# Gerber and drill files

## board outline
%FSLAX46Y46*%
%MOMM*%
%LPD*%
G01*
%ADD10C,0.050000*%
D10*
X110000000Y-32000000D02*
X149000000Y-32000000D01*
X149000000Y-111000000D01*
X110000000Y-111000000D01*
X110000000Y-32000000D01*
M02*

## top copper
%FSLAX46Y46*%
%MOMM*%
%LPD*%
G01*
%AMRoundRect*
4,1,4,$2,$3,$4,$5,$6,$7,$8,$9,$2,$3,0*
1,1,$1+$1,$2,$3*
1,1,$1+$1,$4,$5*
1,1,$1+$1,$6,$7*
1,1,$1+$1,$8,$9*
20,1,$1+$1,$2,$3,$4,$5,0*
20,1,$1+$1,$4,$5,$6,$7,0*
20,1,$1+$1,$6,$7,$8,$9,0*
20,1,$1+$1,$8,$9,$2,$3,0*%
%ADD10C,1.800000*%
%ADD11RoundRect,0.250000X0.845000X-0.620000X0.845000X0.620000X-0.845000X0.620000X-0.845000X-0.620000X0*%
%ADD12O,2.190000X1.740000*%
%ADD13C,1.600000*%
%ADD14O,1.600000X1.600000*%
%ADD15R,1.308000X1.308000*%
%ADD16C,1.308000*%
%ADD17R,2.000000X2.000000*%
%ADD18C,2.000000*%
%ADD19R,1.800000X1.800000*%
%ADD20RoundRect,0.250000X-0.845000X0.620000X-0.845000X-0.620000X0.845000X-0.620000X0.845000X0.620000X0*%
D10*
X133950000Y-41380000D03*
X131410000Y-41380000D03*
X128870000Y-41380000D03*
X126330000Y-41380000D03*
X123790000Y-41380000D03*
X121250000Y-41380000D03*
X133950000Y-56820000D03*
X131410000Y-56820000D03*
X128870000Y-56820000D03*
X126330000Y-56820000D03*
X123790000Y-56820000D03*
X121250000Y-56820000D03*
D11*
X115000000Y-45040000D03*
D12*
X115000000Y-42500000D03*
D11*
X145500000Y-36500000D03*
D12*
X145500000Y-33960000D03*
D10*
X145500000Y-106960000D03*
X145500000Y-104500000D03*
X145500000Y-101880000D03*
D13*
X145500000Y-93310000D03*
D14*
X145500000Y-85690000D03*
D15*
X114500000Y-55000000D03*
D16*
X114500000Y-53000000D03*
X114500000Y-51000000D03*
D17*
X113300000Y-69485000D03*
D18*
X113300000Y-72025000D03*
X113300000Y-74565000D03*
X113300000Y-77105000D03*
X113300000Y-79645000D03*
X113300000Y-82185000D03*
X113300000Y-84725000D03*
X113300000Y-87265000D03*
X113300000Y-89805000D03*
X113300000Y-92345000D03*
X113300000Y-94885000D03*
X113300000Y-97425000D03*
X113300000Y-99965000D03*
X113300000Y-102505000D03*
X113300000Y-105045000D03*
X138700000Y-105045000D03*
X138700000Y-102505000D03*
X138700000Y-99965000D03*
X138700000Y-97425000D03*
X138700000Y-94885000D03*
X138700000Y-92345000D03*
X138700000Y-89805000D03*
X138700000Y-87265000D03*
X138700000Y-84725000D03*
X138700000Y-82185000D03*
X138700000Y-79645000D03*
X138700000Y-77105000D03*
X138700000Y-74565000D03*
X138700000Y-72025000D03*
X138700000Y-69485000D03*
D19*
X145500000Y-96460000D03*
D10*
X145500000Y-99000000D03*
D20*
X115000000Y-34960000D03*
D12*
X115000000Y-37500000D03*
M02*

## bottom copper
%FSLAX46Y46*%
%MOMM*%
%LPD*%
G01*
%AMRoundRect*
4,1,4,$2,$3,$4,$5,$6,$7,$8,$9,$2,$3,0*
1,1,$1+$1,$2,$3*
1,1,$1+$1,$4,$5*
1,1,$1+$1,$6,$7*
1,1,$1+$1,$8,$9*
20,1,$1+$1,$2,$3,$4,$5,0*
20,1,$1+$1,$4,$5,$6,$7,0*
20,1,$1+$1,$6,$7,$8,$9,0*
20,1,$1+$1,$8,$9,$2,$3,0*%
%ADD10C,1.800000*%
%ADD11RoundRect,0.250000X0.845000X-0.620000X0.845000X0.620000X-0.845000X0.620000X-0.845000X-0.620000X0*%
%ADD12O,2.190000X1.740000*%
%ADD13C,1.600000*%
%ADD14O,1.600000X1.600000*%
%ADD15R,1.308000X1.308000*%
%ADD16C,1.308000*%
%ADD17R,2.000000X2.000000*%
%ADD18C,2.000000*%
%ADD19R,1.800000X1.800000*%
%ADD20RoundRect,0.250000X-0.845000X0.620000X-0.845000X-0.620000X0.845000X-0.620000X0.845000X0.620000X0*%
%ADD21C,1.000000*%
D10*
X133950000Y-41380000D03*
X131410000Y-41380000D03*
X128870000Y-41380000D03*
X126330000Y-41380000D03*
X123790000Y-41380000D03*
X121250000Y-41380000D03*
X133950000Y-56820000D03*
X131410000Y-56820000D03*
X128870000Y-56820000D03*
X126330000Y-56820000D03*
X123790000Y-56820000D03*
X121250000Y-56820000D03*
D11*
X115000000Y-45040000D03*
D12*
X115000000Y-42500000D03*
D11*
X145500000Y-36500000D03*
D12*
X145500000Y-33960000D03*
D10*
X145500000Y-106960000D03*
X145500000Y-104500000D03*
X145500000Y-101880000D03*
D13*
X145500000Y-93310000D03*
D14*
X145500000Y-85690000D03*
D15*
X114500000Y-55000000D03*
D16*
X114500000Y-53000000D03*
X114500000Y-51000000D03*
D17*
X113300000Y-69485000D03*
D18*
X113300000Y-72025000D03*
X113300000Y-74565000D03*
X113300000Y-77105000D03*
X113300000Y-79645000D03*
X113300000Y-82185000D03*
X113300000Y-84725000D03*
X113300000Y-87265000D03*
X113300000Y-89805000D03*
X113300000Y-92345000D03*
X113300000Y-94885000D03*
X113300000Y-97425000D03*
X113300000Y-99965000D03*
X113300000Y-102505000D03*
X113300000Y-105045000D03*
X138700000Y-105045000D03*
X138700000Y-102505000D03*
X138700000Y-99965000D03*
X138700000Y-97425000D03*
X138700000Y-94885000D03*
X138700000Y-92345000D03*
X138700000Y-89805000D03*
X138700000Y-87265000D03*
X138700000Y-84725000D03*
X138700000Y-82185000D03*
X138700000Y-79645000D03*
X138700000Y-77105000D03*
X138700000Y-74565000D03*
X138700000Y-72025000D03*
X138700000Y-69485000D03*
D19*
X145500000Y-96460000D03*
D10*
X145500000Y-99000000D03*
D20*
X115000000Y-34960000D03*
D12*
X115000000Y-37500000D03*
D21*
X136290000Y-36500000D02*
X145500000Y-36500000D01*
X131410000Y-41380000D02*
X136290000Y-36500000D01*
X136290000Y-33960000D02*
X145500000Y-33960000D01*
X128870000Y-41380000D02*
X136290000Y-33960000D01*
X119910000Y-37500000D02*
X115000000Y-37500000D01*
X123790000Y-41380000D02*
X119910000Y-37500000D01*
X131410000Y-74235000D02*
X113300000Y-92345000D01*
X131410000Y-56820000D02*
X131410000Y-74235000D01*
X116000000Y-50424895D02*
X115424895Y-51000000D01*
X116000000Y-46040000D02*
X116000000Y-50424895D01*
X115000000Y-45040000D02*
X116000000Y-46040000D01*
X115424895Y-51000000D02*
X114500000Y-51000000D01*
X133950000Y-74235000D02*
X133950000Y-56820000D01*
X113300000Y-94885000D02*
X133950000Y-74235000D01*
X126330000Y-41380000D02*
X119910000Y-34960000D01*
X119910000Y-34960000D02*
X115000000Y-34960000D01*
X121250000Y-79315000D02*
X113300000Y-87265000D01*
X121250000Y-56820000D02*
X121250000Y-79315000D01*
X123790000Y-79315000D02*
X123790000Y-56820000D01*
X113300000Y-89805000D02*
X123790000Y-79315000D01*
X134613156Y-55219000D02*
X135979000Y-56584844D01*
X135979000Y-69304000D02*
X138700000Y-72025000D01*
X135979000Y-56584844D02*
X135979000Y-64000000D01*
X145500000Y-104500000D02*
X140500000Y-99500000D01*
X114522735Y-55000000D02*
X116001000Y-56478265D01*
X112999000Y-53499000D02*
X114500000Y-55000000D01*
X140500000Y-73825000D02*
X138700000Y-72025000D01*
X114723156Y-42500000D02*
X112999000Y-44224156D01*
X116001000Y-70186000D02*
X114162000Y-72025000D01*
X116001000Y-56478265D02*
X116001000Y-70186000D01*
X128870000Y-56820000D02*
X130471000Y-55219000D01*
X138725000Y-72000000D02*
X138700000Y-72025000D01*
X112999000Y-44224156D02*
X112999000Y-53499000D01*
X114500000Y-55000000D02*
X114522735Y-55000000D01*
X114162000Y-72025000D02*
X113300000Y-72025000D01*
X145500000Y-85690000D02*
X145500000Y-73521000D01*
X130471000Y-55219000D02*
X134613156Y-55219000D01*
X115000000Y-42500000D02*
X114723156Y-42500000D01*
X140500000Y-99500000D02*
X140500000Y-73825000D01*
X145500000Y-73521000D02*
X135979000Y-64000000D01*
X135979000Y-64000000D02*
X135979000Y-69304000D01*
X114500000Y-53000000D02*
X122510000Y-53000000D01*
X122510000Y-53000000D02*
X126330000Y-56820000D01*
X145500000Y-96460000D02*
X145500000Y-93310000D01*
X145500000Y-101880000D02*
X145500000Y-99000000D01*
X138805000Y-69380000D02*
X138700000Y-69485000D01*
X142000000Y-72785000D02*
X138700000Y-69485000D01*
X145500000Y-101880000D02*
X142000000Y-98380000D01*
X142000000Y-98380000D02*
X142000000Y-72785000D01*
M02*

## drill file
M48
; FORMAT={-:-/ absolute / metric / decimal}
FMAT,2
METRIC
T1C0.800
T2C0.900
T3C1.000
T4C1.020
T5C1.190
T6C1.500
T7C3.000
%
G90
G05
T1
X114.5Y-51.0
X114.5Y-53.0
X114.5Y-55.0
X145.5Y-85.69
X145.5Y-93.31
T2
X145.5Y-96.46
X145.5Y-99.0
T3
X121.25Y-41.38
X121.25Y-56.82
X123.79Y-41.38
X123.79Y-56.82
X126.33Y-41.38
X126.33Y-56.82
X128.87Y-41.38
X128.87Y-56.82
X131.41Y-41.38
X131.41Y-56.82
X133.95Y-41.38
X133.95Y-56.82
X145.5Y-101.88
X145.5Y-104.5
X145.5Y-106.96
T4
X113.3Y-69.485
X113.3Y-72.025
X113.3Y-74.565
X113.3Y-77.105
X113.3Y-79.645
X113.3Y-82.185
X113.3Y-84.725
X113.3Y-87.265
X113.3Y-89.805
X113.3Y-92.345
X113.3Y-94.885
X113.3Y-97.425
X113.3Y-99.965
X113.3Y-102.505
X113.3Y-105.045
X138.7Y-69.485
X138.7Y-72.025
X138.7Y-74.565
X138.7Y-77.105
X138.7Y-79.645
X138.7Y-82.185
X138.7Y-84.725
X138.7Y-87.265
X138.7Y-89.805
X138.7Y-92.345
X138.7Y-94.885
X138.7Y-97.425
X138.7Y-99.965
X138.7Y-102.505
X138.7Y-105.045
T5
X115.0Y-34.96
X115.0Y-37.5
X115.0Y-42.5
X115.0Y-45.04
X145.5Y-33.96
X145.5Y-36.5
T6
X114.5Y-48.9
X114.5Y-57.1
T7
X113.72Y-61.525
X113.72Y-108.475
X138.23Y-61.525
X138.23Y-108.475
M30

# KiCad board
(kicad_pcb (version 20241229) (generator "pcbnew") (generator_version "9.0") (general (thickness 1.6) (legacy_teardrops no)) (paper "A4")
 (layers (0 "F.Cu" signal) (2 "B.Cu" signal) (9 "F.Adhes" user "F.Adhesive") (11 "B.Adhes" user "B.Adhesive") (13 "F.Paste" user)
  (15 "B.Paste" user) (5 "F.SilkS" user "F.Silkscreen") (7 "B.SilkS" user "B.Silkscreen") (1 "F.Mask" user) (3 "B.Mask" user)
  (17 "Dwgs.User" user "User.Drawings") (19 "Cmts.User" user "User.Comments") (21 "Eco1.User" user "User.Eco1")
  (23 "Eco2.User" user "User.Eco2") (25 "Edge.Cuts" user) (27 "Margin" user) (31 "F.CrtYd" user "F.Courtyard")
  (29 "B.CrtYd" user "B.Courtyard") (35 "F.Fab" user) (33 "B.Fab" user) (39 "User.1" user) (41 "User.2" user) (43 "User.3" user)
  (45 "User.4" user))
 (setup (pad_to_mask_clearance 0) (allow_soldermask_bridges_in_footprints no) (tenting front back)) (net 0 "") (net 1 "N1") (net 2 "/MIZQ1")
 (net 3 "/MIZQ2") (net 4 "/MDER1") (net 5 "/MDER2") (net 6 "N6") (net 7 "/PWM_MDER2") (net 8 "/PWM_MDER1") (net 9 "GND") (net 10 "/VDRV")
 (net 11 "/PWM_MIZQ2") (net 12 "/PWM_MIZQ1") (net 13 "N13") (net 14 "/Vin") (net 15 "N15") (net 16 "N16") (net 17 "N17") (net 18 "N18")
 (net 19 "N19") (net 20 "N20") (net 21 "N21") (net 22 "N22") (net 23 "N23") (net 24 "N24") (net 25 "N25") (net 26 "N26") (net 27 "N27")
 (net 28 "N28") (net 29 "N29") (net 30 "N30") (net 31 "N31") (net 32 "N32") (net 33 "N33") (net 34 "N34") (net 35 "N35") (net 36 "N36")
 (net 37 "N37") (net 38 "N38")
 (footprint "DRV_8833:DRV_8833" (layer "F.Cu") (at 119.6 39.85 -90)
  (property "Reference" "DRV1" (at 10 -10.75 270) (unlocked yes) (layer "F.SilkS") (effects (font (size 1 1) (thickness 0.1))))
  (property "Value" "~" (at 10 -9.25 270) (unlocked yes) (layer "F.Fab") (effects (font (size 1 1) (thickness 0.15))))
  (pad "1" thru_hole circle (at 1.53 -14.35 270) (size 1.8 1.8) (drill 1) (layers "*.Cu" "*.Mask") (remove_unused_layers no) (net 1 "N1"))
  (pad "2" thru_hole circle (at 1.53 -11.81 270) (size 1.8 1.8) (drill 1) (layers "*.Cu" "*.Mask") (remove_unused_layers no)
   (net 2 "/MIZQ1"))
  (pad "3" thru_hole circle (at 1.53 -9.27 270) (size 1.8 1.8) (drill 1) (layers "*.Cu" "*.Mask") (remove_unused_layers no) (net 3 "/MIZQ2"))
  (pad "4" thru_hole circle (at 1.53 -6.73 270) (size 1.8 1.8) (drill 1) (layers "*.Cu" "*.Mask") (remove_unused_layers no) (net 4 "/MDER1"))
  (pad "5" thru_hole circle (at 1.53 -4.19 270) (size 1.8 1.8) (drill 1) (layers "*.Cu" "*.Mask") (remove_unused_layers no) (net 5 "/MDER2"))
  (pad "6" thru_hole circle (at 1.53 -1.65 270) (size 1.8 1.8) (drill 1) (layers "*.Cu" "*.Mask") (remove_unused_layers no) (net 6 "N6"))
  (pad "7" thru_hole circle (at 16.97 -14.35 270) (size 1.8 1.8) (drill 1) (layers "*.Cu" "*.Mask") (remove_unused_layers no)
   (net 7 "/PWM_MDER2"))
  (pad "8" thru_hole circle (at 16.97 -11.81 270) (size 1.8 1.8) (drill 1) (layers "*.Cu" "*.Mask") (remove_unused_layers no)
   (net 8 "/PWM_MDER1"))
  (pad "9" thru_hole circle (at 16.97 -9.27 270) (size 1.8 1.8) (drill 1) (layers "*.Cu" "*.Mask") (remove_unused_layers no) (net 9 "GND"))
  (pad "10" thru_hole circle (at 16.97 -6.73 270) (size 1.8 1.8) (drill 1) (layers "*.Cu" "*.Mask") (remove_unused_layers no)
   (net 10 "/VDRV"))
  (pad "11" thru_hole circle (at 16.97 -4.19 270) (size 1.8 1.8) (drill 1) (layers "*.Cu" "*.Mask") (remove_unused_layers no)
   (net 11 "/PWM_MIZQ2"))
  (pad "12" thru_hole circle (at 16.97 -1.65 270) (size 1.8 1.8) (drill 1) (layers "*.Cu" "*.Mask") (remove_unused_layers no)
   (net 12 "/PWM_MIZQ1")))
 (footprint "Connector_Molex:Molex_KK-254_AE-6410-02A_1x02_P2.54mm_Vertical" (layer "F.Cu") (at 115 45.04 90)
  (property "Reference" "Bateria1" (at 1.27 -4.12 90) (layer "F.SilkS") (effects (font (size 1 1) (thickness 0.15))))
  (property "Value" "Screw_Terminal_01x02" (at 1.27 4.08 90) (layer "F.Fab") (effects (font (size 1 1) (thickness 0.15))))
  (pad "1" thru_hole roundrect (at 0 0 90) (size 1.74 2.19) (drill 1.19) (layers "*.Cu" "*.Mask") (remove_unused_layers no)
   (roundrect_rratio 0.143678) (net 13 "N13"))
  (pad "2" thru_hole oval (at 2.54 0 90) (size 1.74 2.19) (drill 1.19) (layers "*.Cu" "*.Mask") (remove_unused_layers no) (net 9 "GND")))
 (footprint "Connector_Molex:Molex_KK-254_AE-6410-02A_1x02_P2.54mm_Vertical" (layer "F.Cu") (at 145.5 36.5 90)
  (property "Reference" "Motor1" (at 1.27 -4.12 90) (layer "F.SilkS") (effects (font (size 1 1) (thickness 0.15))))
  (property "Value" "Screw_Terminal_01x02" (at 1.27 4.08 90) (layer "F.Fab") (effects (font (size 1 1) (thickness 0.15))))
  (pad "1" thru_hole roundrect (at 0 0 90) (size 1.74 2.19) (drill 1.19) (layers "*.Cu" "*.Mask") (remove_unused_layers no)
   (roundrect_rratio 0.143678) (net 2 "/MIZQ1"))
  (pad "2" thru_hole oval (at 2.54 0 90) (size 1.74 2.19) (drill 1.19) (layers "*.Cu" "*.Mask") (remove_unused_layers no) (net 3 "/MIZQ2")))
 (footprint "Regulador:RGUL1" (layer "F.Cu") (at 145.5 104.5 90)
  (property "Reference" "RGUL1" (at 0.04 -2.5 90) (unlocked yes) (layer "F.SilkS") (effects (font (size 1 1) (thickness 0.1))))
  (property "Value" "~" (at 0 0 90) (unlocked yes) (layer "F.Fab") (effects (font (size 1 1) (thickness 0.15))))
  (pad "1" thru_hole circle (at -2.46 0 90) (size 1.8 1.8) (drill 1) (layers "*.Cu" "*.Mask") (remove_unused_layers no) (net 10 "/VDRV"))
  (pad "2" thru_hole circle (at 0 0 90) (size 1.8 1.8) (drill 1) (layers "*.Cu" "*.Mask") (remove_unused_layers no) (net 9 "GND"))
  (pad "3" thru_hole circle (at 2.62 0 90) (size 1.8 1.8) (drill 1) (layers "*.Cu" "*.Mask") (remove_unused_layers no) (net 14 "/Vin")))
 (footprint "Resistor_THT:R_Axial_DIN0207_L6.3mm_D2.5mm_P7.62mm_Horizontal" (layer "F.Cu") (at 145.5 93.31 90)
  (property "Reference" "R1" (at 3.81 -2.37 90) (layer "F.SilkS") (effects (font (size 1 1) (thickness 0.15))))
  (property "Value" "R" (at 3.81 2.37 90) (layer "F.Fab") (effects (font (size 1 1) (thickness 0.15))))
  (pad "1" thru_hole circle (at 0 0 90) (size 1.6 1.6) (drill 0.8) (layers "*.Cu" "*.Mask") (remove_unused_layers no) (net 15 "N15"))
  (pad "2" thru_hole oval (at 7.62 0 90) (size 1.6 1.6) (drill 0.8) (layers "*.Cu" "*.Mask") (remove_unused_layers no) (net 9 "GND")))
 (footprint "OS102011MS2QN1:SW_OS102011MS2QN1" (layer "F.Cu") (at 114.5 53 90)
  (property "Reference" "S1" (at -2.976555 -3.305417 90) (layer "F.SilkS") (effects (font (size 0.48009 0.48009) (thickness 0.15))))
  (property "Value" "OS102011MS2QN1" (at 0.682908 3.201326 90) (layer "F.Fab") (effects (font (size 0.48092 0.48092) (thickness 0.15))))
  (pad "" np_thru_hole circle (at -4.1 0 90) (size 1.5 1.5) (drill 1.5) (layers "*.Cu" "*.Mask"))
  (pad "" np_thru_hole circle (at 4.1 0 90) (size 1.5 1.5) (drill 1.5) (layers "*.Cu" "*.Mask"))
  (pad "1" thru_hole rect (at -2 0 90) (size 1.308 1.308) (drill 0.8) (layers "*.Cu" "*.Mask") (remove_unused_layers no) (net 9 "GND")
   (solder_mask_margin 0.102))
  (pad "2" thru_hole circle (at 0 0 90) (size 1.308 1.308) (drill 0.8) (layers "*.Cu" "*.Mask") (remove_unused_layers no) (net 10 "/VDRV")
   (solder_mask_margin 0.102))
  (pad "3" thru_hole circle (at 2 0 90) (size 1.308 1.308) (drill 0.8) (layers "*.Cu" "*.Mask") (remove_unused_layers no) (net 13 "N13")
   (solder_mask_margin 0.102)))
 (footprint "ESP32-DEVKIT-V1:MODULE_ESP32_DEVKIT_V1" (layer "F.Cu") (at 126 85)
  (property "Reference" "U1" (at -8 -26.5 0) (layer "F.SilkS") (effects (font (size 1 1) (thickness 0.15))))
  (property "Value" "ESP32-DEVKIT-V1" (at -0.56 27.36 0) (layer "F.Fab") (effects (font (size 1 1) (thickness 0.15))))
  (pad "" np_thru_hole circle (at -12.28 -23.475) (size 3 3) (drill 3) (layers "*.Cu" "*.Mask"))
  (pad "" np_thru_hole circle (at -12.28 23.475) (size 3 3) (drill 3) (layers "*.Cu" "*.Mask"))
  (pad "" np_thru_hole circle (at 12.23 -23.475) (size 3 3) (drill 3) (layers "*.Cu" "*.Mask"))
  (pad "" np_thru_hole circle (at 12.23 23.475) (size 3 3) (drill 3) (layers "*.Cu" "*.Mask"))
  (pad "1" thru_hole rect (at -12.7 -15.515) (size 2 2) (drill 1.02) (layers "*.Cu" "*.Mask") (remove_unused_layers no) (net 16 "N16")
   (solder_mask_margin 0.102))
  (pad "2" thru_hole circle (at -12.7 -12.975) (size 2 2) (drill 1.02) (layers "*.Cu" "*.Mask") (remove_unused_layers no) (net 9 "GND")
   (solder_mask_margin 0.102))
  (pad "3" thru_hole circle (at -12.7 -10.435) (size 2 2) (drill 1.02) (layers "*.Cu" "*.Mask") (remove_unused_layers no) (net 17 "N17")
   (solder_mask_margin 0.102))
  (pad "4" thru_hole circle (at -12.7 -7.895) (size 2 2) (drill 1.02) (layers "*.Cu" "*.Mask") (remove_unused_layers no) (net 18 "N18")
   (solder_mask_margin 0.102))
  (pad "5" thru_hole circle (at -12.7 -5.355) (size 2 2) (drill 1.02) (layers "*.Cu" "*.Mask") (remove_unused_layers no) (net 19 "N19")
   (solder_mask_margin 0.102))
  (pad "6" thru_hole circle (at -12.7 -2.815) (size 2 2) (drill 1.02) (layers "*.Cu" "*.Mask") (remove_unused_layers no) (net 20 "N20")
   (solder_mask_margin 0.102))
  (pad "7" thru_hole circle (at -12.7 -0.275) (size 2 2) (drill 1.02) (layers "*.Cu" "*.Mask") (remove_unused_layers no) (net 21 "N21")
   (solder_mask_margin 0.102))
  (pad "8" thru_hole circle (at -12.7 2.265) (size 2 2) (drill 1.02) (layers "*.Cu" "*.Mask") (remove_unused_layers no)
   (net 12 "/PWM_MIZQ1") (solder_mask_margin 0.102))
  (pad "9" thru_hole circle (at -12.7 4.805) (size 2 2) (drill 1.02) (layers "*.Cu" "*.Mask") (remove_unused_layers no)
   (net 11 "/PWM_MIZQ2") (solder_mask_margin 0.102))
  (pad "10" thru_hole circle (at -12.7 7.345) (size 2 2) (drill 1.02) (layers "*.Cu" "*.Mask") (remove_unused_layers no)
   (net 8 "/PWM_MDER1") (solder_mask_margin 0.102))
  (pad "11" thru_hole circle (at -12.7 9.885) (size 2 2) (drill 1.02) (layers "*.Cu" "*.Mask") (remove_unused_layers no)
   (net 7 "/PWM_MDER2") (solder_mask_margin 0.102))
  (pad "12" thru_hole circle (at -12.7 12.425) (size 2 2) (drill 1.02) (layers "*.Cu" "*.Mask") (remove_unused_layers no) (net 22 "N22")
   (solder_mask_margin 0.102))
  (pad "13" thru_hole circle (at -12.7 14.965) (size 2 2) (drill 1.02) (layers "*.Cu" "*.Mask") (remove_unused_layers no) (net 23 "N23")
   (solder_mask_margin 0.102))
  (pad "14" thru_hole circle (at -12.7 17.505) (size 2 2) (drill 1.02) (layers "*.Cu" "*.Mask") (remove_unused_layers no) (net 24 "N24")
   (solder_mask_margin 0.102))
  (pad "15" thru_hole circle (at -12.7 20.045) (size 2 2) (drill 1.02) (layers "*.Cu" "*.Mask") (remove_unused_layers no) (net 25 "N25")
   (solder_mask_margin 0.102))
  (pad "16" thru_hole circle (at 12.7 20.045) (size 2 2) (drill 1.02) (layers "*.Cu" "*.Mask") (remove_unused_layers no) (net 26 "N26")
   (solder_mask_margin 0.102))
  (pad "17" thru_hole circle (at 12.7 17.505) (size 2 2) (drill 1.02) (layers "*.Cu" "*.Mask") (remove_unused_layers no) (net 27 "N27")
   (solder_mask_margin 0.102))
  (pad "18" thru_hole circle (at 12.7 14.965) (size 2 2) (drill 1.02) (layers "*.Cu" "*.Mask") (remove_unused_layers no) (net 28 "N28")
   (solder_mask_margin 0.102))
  (pad "19" thru_hole circle (at 12.7 12.425) (size 2 2) (drill 1.02) (layers "*.Cu" "*.Mask") (remove_unused_layers no) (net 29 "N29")
   (solder_mask_margin 0.102))
  (pad "20" thru_hole circle (at 12.7 9.885) (size 2 2) (drill 1.02) (layers "*.Cu" "*.Mask") (remove_unused_layers no) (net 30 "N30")
   (solder_mask_margin 0.102))
  (pad "21" thru_hole circle (at 12.7 7.345) (size 2 2) (drill 1.02) (layers "*.Cu" "*.Mask") (remove_unused_layers no) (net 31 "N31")
   (solder_mask_margin 0.102))
  (pad "22" thru_hole circle (at 12.7 4.805) (size 2 2) (drill 1.02) (layers "*.Cu" "*.Mask") (remove_unused_layers no) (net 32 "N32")
   (solder_mask_margin 0.102))
  (pad "23" thru_hole circle (at 12.7 2.265) (size 2 2) (drill 1.02) (layers "*.Cu" "*.Mask") (remove_unused_layers no) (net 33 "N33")
   (solder_mask_margin 0.102))
  (pad "24" thru_hole circle (at 12.7 -0.275) (size 2 2) (drill 1.02) (layers "*.Cu" "*.Mask") (remove_unused_layers no) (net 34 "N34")
   (solder_mask_margin 0.102))
  (pad "25" thru_hole circle (at 12.7 -2.815) (size 2 2) (drill 1.02) (layers "*.Cu" "*.Mask") (remove_unused_layers no) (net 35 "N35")
   (solder_mask_margin 0.102))
  (pad "26" thru_hole circle (at 12.7 -5.355) (size 2 2) (drill 1.02) (layers "*.Cu" "*.Mask") (remove_unused_layers no) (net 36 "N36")
   (solder_mask_margin 0.102))
  (pad "27" thru_hole circle (at 12.7 -7.895) (size 2 2) (drill 1.02) (layers "*.Cu" "*.Mask") (remove_unused_layers no) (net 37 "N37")
   (solder_mask_margin 0.102))
  (pad "28" thru_hole circle (at 12.7 -10.435) (size 2 2) (drill 1.02) (layers "*.Cu" "*.Mask") (remove_unused_layers no) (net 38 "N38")
   (solder_mask_margin 0.102))
  (pad "29" thru_hole circle (at 12.7 -12.975) (size 2 2) (drill 1.02) (layers "*.Cu" "*.Mask") (remove_unused_layers no) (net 9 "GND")
   (solder_mask_margin 0.102))
  (pad "30" thru_hole circle (at 12.7 -15.515) (size 2 2) (drill 1.02) (layers "*.Cu" "*.Mask") (remove_unused_layers no) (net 14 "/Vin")
   (solder_mask_margin 0.102))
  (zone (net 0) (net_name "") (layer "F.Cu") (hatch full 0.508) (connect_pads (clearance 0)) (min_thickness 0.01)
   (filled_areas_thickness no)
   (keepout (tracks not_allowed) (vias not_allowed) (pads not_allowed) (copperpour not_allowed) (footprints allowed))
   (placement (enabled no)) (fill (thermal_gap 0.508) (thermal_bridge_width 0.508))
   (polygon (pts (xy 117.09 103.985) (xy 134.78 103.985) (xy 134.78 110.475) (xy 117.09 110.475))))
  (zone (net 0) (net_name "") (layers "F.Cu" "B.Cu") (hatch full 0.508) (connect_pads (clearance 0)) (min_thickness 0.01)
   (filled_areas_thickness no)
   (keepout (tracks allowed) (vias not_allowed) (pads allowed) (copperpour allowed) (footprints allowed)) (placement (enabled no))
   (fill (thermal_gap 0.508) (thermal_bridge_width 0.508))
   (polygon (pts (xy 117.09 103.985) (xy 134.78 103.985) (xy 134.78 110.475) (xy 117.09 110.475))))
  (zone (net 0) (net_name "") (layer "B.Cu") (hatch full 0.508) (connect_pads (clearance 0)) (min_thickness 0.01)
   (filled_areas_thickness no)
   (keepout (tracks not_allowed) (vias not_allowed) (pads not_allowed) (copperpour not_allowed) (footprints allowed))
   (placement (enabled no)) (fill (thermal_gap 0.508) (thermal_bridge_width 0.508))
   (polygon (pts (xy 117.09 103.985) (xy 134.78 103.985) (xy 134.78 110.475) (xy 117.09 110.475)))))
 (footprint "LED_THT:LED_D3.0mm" (layer "F.Cu") (at 145.5 96.46 -90)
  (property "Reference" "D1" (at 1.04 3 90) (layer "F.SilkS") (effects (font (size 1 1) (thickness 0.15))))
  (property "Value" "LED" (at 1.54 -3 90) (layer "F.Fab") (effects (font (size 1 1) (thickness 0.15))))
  (pad "1" thru_hole rect (at 0 0 270) (size 1.8 1.8) (drill 0.9) (layers "*.Cu" "*.Mask") (remove_unused_layers no) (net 15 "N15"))
  (pad "2" thru_hole circle (at 2.54 0 270) (size 1.8 1.8) (drill 0.9) (layers "*.Cu" "*.Mask") (remove_unused_layers no) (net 14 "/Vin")))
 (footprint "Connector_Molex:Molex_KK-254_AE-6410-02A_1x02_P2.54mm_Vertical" (layer "F.Cu") (at 115 34.96 -90)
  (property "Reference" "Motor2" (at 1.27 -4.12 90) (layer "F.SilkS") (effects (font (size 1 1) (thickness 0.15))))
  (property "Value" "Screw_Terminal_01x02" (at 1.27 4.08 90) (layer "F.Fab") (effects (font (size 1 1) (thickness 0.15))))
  (pad "1" thru_hole roundrect (at 0 0 270) (size 1.74 2.19) (drill 1.19) (layers "*.Cu" "*.Mask") (remove_unused_layers no)
   (roundrect_rratio 0.143678) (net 4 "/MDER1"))
  (pad "2" thru_hole oval (at 2.54 0 270) (size 1.74 2.19) (drill 1.19) (layers "*.Cu" "*.Mask") (remove_unused_layers no) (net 5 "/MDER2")))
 (gr_rect (start 110 32) (end 149 111) (stroke (width 0.05) (type default)) (fill no) (layer "Edge.Cuts"))
 (segment (start 136.29 36.5) (end 145.5 36.5) (width 1) (layer "B.Cu") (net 2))
 (segment (start 131.41 41.38) (end 136.29 36.5) (width 1) (layer "B.Cu") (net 2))
 (segment (start 136.29 33.96) (end 145.5 33.96) (width 1) (layer "B.Cu") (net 3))
 (segment (start 128.87 41.38) (end 136.29 33.96) (width 1) (layer "B.Cu") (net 3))
 (segment (start 119.91 37.5) (end 115 37.5) (width 1) (layer "B.Cu") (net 5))
 (segment (start 123.79 41.38) (end 119.91 37.5) (width 1) (layer "B.Cu") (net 5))
 (segment (start 131.41 74.235) (end 113.3 92.345) (width 1) (layer "B.Cu") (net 8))
 (segment (start 131.41 56.82) (end 131.41 74.235) (width 1) (layer "B.Cu") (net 8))
 (segment (start 116 50.424895) (end 115.424895 51) (width 1) (layer "B.Cu") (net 13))
 (segment (start 116 46.04) (end 116 50.424895) (width 1) (layer "B.Cu") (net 13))
 (segment (start 115 45.04) (end 116 46.04) (width 1) (layer "B.Cu") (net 13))
 (segment (start 115.424895 51) (end 114.5 51) (width 1) (layer "B.Cu") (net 13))
 (segment (start 133.95 74.235) (end 133.95 56.82) (width 1) (layer "B.Cu") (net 7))
 (segment (start 113.3 94.885) (end 133.95 74.235) (width 1) (layer "B.Cu") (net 7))
 (segment (start 126.33 41.38) (end 119.91 34.96) (width 1) (layer "B.Cu") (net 4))
 (segment (start 119.91 34.96) (end 115 34.96) (width 1) (layer "B.Cu") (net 4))
 (segment (start 121.25 79.315) (end 113.3 87.265) (width 1) (layer "B.Cu") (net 12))
 (segment (start 121.25 56.82) (end 121.25 79.315) (width 1) (layer "B.Cu") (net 12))
 (segment (start 123.79 79.315) (end 123.79 56.82) (width 1) (layer "B.Cu") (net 11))
 (segment (start 113.3 89.805) (end 123.79 79.315) (width 1) (layer "B.Cu") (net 11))
 (segment (start 134.613156 55.219) (end 135.979 56.584844) (width 1) (layer "B.Cu") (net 9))
 (segment (start 135.979 69.304) (end 138.7 72.025) (width 1) (layer "B.Cu") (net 9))
 (segment (start 135.979 56.584844) (end 135.979 64) (width 1) (layer "B.Cu") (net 9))
 (segment (start 145.5 104.5) (end 140.5 99.5) (width 1) (layer "B.Cu") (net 9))
 (segment (start 114.522735 55) (end 116.001 56.478265) (width 1) (layer "B.Cu") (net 9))
 (segment (start 112.999 53.499) (end 114.5 55) (width 1) (layer "B.Cu") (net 9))
 (segment (start 140.5 73.825) (end 138.7 72.025) (width 1) (layer "B.Cu") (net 9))
 (segment (start 114.723156 42.5) (end 112.999 44.224156) (width 1) (layer "B.Cu") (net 9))
 (segment (start 116.001 70.186) (end 114.162 72.025) (width 1) (layer "B.Cu") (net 9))
 (segment (start 116.001 56.478265) (end 116.001 70.186) (width 1) (layer "B.Cu") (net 9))
 (segment (start 128.87 56.82) (end 130.471 55.219) (width 1) (layer "B.Cu") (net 9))
 (segment (start 138.725 72) (end 138.7 72.025) (width 1) (layer "B.Cu") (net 9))
 (segment (start 112.999 44.224156) (end 112.999 53.499) (width 1) (layer "B.Cu") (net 9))
 (segment (start 114.5 55) (end 114.522735 55) (width 1) (layer "B.Cu") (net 9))
 (segment (start 114.162 72.025) (end 113.3 72.025) (width 1) (layer "B.Cu") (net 9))
 (segment (start 145.5 85.69) (end 145.5 73.521) (width 1) (layer "B.Cu") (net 9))
 (segment (start 130.471 55.219) (end 134.613156 55.219) (width 1) (layer "B.Cu") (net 9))
 (segment (start 115 42.5) (end 114.723156 42.5) (width 1) (layer "B.Cu") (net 9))
 (segment (start 140.5 99.5) (end 140.5 73.825) (width 1) (layer "B.Cu") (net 9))
 (segment (start 145.5 73.521) (end 135.979 64) (width 1) (layer "B.Cu") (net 9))
 (segment (start 135.979 64) (end 135.979 69.304) (width 1) (layer "B.Cu") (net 9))
 (segment (start 114.5 53) (end 122.51 53) (width 1) (layer "B.Cu") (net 10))
 (segment (start 122.51 53) (end 126.33 56.82) (width 1) (layer "B.Cu") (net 10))
 (segment (start 145.5 96.46) (end 145.5 93.31) (width 1) (layer "B.Cu") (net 15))
 (segment (start 145.5 101.88) (end 145.5 99) (width 1) (layer "B.Cu") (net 14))
 (segment (start 138.805 69.38) (end 138.7 69.485) (width 1) (layer "B.Cu") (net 14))
 (segment (start 142 72.785) (end 138.7 69.485) (width 1) (layer "B.Cu") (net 14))
 (segment (start 145.5 101.88) (end 142 98.38) (width 1) (layer "B.Cu") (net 14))
 (segment (start 142 98.38) (end 142 72.785) (width 1) (layer "B.Cu") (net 14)))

